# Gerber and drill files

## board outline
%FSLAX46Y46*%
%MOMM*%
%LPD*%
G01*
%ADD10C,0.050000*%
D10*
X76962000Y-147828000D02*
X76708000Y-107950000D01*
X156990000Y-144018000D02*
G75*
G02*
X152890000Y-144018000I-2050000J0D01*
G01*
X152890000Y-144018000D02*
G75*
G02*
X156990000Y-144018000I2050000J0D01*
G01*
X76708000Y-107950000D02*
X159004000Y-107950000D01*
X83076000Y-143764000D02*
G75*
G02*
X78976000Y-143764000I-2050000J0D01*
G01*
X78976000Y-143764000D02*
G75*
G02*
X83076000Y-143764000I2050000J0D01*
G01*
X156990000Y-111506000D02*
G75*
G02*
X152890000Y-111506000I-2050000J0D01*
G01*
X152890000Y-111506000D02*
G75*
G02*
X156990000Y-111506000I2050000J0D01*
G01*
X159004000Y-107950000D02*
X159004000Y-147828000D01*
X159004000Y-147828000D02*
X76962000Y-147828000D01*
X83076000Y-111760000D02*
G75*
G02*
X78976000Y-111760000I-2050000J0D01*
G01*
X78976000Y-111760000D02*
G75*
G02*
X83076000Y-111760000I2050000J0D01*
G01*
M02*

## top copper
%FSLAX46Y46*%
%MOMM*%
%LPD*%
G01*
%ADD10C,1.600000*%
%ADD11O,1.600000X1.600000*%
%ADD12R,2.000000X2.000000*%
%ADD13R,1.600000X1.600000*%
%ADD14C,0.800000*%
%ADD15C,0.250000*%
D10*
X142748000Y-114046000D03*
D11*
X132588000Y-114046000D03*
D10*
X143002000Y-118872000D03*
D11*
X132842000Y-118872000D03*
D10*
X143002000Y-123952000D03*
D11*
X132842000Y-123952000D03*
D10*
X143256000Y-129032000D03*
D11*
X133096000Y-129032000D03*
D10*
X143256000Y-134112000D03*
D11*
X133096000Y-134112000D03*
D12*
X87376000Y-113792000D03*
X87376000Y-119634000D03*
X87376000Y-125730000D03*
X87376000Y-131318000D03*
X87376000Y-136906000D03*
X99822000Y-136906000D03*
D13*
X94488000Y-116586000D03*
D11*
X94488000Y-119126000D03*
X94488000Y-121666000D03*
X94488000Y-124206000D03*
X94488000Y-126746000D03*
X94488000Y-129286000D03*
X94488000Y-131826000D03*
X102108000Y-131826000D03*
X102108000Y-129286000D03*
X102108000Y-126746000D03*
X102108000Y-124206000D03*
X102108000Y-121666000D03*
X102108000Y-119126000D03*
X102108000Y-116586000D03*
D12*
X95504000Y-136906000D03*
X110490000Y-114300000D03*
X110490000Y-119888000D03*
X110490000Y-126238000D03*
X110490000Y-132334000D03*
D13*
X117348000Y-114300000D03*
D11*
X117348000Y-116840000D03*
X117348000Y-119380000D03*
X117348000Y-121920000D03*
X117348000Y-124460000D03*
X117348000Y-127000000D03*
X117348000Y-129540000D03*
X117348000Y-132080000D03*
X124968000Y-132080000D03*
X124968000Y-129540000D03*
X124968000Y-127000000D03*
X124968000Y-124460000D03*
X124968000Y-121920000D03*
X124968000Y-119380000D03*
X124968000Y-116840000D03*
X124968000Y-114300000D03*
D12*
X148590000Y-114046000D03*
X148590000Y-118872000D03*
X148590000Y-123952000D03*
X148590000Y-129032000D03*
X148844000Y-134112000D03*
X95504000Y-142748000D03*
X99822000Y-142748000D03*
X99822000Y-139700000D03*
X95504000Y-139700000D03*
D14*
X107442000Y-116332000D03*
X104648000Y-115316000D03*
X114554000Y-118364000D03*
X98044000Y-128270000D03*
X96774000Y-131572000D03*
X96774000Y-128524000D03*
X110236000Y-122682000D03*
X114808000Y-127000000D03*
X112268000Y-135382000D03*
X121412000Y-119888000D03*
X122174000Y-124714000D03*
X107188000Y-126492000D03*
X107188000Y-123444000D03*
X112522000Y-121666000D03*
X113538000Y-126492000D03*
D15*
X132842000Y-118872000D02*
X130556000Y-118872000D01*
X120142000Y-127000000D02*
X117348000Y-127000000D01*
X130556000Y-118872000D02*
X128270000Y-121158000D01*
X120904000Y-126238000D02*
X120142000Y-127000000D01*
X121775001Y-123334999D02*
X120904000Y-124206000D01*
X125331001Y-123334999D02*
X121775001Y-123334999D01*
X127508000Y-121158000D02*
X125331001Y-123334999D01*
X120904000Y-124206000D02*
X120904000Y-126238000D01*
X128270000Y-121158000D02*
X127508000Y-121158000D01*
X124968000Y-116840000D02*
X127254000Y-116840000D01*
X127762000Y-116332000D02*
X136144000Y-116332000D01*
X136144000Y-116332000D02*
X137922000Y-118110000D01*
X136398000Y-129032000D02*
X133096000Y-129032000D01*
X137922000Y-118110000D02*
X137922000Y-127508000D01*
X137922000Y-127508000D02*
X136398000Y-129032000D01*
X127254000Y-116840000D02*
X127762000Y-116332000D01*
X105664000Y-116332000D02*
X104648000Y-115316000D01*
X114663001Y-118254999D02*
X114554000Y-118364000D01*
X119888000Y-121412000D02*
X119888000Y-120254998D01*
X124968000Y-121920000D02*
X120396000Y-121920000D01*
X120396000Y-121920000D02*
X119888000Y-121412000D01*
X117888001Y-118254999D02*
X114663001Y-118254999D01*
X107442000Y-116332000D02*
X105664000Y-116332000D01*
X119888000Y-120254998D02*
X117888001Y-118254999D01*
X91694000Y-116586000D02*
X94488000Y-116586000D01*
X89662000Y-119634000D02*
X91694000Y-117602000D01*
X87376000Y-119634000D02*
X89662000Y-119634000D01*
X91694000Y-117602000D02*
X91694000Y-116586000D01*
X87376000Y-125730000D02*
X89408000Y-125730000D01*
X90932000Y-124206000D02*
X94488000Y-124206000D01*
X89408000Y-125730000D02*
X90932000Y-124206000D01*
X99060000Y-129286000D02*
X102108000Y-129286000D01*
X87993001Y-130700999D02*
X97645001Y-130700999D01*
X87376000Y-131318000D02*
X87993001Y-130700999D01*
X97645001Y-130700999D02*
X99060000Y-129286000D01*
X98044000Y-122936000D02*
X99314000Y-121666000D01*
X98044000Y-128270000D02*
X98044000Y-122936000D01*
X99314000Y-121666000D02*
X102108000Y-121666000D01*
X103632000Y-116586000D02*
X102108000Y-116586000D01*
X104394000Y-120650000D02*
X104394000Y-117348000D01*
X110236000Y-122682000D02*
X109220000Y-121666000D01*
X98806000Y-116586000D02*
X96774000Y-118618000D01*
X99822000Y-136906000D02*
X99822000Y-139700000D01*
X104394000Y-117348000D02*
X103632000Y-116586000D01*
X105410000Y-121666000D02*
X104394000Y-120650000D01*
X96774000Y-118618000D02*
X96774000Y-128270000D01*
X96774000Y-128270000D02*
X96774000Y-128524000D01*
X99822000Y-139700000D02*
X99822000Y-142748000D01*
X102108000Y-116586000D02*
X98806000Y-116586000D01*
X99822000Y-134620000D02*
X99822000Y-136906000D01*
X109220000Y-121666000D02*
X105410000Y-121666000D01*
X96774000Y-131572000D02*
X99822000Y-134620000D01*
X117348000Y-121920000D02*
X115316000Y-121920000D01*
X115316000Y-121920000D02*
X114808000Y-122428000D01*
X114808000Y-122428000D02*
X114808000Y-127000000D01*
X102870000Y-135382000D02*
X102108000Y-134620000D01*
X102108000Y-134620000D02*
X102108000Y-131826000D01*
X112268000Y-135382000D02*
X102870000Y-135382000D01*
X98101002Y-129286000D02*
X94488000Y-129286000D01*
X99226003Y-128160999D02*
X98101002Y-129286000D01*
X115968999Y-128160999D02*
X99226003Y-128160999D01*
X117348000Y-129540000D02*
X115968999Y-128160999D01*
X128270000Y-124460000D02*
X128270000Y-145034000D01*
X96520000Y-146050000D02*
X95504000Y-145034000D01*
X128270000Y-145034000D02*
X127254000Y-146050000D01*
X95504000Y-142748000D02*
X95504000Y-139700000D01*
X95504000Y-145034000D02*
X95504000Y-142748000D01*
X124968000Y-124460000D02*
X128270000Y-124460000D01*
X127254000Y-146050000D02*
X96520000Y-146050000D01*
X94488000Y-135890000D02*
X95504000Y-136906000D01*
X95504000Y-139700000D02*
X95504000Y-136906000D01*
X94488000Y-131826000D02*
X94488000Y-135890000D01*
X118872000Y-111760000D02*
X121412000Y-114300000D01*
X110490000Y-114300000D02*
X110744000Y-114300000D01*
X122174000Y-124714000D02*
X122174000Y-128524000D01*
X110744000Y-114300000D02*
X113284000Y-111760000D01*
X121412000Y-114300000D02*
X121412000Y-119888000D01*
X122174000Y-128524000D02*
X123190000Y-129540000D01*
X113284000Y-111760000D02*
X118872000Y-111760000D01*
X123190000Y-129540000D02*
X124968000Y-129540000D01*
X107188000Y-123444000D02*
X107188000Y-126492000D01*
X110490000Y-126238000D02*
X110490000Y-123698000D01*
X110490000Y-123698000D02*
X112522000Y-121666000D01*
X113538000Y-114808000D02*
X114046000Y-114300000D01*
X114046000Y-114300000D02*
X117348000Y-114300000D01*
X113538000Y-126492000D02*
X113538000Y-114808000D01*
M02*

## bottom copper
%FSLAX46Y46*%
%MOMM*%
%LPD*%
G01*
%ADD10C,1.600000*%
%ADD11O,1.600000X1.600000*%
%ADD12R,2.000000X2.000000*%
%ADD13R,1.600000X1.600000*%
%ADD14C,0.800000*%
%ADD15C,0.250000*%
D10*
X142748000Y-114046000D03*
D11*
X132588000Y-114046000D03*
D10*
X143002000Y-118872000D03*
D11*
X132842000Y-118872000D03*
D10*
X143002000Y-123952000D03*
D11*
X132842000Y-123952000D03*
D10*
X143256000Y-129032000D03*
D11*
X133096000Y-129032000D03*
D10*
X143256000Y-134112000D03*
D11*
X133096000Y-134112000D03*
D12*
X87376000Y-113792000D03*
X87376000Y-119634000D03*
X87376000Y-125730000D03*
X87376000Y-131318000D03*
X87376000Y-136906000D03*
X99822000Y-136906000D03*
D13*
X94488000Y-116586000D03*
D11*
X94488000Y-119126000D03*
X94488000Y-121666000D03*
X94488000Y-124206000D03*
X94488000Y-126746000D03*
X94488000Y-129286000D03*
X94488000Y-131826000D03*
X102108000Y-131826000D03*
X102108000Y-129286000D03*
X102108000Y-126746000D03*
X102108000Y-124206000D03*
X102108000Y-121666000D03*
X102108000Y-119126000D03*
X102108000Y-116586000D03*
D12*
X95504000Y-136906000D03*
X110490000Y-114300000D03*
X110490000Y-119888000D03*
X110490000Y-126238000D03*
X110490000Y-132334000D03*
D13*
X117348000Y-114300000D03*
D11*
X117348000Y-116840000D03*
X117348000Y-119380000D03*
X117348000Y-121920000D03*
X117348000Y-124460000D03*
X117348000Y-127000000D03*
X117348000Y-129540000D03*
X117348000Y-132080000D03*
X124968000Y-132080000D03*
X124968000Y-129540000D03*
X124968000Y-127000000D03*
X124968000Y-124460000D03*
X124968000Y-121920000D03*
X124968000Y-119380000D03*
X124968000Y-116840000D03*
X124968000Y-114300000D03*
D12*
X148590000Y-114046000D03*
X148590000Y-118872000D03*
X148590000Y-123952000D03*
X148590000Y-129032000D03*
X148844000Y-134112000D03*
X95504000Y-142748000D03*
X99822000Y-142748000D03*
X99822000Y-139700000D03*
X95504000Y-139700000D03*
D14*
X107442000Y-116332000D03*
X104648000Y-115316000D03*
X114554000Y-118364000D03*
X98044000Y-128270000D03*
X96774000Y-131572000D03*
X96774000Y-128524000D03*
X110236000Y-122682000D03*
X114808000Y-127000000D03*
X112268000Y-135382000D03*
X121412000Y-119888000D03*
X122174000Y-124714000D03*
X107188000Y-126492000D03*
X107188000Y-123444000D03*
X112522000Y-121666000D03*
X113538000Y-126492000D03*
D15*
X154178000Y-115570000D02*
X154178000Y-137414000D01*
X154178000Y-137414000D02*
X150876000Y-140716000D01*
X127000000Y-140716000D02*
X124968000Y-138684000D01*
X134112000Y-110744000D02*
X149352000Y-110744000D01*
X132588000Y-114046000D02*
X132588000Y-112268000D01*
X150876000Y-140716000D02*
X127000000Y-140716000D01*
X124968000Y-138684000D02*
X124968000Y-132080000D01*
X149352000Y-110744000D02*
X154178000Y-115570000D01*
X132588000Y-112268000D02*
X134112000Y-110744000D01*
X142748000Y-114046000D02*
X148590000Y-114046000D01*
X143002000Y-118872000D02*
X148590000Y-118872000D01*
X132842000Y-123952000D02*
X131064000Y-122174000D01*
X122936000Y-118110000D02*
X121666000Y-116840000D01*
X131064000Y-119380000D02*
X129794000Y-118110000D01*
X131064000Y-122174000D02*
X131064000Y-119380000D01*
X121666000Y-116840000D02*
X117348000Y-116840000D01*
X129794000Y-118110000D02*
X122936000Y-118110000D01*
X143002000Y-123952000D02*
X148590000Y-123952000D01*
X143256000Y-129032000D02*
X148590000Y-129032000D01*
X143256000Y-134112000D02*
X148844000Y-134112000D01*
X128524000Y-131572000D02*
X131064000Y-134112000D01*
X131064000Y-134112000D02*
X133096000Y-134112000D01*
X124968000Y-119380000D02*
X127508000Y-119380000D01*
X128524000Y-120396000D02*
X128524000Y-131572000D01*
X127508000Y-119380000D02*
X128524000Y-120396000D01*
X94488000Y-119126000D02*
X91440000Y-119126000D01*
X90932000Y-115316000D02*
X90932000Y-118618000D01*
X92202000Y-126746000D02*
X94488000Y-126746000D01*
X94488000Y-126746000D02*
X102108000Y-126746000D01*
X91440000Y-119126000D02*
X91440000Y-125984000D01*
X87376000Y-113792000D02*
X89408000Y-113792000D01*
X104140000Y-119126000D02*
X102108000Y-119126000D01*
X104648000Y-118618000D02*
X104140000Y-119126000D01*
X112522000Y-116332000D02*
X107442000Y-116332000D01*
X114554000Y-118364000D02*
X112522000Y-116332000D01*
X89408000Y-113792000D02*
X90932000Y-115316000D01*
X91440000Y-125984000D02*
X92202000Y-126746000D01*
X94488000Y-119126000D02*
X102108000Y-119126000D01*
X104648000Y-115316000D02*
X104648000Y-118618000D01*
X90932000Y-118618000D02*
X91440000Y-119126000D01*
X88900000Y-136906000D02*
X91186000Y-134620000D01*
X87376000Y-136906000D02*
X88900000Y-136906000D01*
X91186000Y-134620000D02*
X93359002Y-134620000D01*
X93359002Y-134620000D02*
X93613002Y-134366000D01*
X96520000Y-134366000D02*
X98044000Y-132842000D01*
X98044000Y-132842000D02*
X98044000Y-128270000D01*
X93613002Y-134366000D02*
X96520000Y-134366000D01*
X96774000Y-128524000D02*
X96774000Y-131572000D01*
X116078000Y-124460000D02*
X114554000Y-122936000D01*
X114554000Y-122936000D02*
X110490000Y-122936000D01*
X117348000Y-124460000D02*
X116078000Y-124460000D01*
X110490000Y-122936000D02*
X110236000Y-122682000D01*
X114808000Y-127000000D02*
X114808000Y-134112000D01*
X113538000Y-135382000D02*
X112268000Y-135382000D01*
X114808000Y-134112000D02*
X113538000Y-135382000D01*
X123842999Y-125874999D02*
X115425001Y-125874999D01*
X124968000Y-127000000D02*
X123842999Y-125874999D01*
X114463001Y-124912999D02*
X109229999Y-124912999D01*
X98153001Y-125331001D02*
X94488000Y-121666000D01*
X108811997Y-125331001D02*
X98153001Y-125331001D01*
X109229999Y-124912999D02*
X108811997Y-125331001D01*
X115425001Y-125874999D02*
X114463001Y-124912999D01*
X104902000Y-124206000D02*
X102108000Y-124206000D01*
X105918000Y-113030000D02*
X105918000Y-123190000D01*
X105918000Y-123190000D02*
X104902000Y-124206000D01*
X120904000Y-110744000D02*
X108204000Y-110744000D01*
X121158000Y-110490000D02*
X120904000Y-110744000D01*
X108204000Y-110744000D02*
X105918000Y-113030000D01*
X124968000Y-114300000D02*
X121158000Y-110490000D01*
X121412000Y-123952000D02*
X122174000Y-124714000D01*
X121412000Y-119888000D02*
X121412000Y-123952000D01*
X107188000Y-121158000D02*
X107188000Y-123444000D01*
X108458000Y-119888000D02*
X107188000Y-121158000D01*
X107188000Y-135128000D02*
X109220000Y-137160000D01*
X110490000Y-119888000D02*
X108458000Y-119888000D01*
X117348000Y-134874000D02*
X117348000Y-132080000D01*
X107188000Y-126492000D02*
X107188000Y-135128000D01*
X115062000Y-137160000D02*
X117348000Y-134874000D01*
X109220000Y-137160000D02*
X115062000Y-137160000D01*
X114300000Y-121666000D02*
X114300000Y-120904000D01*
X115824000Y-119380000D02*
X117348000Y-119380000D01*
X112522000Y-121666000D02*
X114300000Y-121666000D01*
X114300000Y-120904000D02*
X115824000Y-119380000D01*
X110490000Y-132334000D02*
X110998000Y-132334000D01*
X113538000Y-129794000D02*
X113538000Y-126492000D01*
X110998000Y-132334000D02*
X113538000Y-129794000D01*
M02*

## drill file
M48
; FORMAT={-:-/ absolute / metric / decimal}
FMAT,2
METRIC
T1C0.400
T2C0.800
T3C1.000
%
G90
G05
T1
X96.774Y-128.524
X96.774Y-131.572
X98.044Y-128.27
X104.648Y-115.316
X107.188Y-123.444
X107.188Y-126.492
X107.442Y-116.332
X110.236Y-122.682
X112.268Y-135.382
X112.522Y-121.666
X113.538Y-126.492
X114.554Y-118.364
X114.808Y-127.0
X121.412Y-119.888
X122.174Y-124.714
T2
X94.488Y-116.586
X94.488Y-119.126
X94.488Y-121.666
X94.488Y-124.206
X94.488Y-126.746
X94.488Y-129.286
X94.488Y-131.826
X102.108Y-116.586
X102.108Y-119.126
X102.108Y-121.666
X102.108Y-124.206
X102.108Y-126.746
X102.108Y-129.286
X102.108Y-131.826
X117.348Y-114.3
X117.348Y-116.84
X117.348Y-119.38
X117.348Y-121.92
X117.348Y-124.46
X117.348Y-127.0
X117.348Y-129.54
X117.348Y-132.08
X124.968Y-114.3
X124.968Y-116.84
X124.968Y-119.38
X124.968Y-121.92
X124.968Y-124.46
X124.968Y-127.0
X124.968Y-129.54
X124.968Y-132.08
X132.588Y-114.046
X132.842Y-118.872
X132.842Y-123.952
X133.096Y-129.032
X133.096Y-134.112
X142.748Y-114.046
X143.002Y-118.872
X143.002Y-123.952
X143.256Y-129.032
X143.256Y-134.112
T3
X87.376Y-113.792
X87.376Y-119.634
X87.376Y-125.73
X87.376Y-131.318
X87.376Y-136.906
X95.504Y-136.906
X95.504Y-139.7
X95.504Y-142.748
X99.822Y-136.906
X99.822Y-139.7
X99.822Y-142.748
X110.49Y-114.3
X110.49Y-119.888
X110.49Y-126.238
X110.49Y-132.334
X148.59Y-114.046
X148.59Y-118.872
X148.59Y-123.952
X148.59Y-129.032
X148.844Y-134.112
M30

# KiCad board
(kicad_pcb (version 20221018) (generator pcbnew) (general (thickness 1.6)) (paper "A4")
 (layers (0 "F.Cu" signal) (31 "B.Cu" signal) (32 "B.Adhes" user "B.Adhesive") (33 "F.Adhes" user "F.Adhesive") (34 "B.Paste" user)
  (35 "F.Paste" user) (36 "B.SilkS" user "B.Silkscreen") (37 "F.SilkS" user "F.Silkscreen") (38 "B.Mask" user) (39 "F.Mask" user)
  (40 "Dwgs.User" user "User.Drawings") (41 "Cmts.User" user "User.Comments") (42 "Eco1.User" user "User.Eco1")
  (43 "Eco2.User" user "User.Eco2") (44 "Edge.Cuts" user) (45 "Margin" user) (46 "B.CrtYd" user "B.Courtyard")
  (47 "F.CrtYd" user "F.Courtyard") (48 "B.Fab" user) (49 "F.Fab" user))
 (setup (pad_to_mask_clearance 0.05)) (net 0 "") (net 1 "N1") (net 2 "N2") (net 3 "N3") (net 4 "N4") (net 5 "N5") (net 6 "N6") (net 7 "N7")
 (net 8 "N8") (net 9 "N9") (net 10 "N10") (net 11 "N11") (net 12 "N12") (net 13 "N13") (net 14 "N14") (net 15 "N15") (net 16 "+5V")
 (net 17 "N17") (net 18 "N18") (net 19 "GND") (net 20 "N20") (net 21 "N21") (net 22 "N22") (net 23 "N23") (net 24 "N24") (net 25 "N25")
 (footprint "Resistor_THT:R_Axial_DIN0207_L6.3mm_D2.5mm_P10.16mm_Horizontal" (layer "F.Cu") (at 142.748 114.046 180)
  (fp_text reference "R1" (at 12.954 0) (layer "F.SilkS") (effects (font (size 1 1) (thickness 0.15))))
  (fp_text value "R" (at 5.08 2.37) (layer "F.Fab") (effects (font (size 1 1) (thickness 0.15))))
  (pad "1" thru_hole circle (at 0 0 180) (size 1.6 1.6) (drill 0.8) (layers "*.Cu" "*.Mask") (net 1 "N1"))
  (pad "2" thru_hole oval (at 10.16 0 180) (size 1.6 1.6) (drill 0.8) (layers "*.Cu" "*.Mask") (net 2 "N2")))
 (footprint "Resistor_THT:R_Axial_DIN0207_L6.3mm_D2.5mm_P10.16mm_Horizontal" (layer "F.Cu") (at 143.002 118.872 180)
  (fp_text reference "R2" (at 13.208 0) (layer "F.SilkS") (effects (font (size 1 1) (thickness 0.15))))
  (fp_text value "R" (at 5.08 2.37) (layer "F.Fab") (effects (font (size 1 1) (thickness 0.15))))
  (pad "1" thru_hole circle (at 0 0 180) (size 1.6 1.6) (drill 0.8) (layers "*.Cu" "*.Mask") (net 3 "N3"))
  (pad "2" thru_hole oval (at 10.16 0 180) (size 1.6 1.6) (drill 0.8) (layers "*.Cu" "*.Mask") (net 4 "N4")))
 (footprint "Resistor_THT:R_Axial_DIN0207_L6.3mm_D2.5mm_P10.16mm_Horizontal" (layer "F.Cu") (at 143.002 123.952 180)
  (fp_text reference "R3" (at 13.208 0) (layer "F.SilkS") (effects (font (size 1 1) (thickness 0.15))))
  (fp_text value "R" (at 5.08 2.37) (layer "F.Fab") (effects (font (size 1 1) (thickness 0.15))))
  (pad "1" thru_hole circle (at 0 0 180) (size 1.6 1.6) (drill 0.8) (layers "*.Cu" "*.Mask") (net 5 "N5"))
  (pad "2" thru_hole oval (at 10.16 0 180) (size 1.6 1.6) (drill 0.8) (layers "*.Cu" "*.Mask") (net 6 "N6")))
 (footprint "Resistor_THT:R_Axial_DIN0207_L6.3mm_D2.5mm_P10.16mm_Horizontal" (layer "F.Cu") (at 143.256 129.032 180)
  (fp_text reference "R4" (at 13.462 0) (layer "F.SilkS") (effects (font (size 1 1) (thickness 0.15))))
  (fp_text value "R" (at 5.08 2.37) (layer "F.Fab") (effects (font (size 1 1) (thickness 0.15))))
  (pad "1" thru_hole circle (at 0 0 180) (size 1.6 1.6) (drill 0.8) (layers "*.Cu" "*.Mask") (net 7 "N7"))
  (pad "2" thru_hole oval (at 10.16 0 180) (size 1.6 1.6) (drill 0.8) (layers "*.Cu" "*.Mask") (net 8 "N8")))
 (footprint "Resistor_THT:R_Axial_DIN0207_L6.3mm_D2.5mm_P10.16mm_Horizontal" (layer "F.Cu") (at 143.256 134.112 180)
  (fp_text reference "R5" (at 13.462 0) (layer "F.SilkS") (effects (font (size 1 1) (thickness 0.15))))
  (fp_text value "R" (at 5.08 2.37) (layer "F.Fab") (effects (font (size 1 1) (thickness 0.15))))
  (pad "1" thru_hole circle (at 0 0 180) (size 1.6 1.6) (drill 0.8) (layers "*.Cu" "*.Mask") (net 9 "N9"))
  (pad "2" thru_hole oval (at 10.16 0 180) (size 1.6 1.6) (drill 0.8) (layers "*.Cu" "*.Mask") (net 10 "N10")))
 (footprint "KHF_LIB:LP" (layer "F.Cu") (at 87.376 113.792)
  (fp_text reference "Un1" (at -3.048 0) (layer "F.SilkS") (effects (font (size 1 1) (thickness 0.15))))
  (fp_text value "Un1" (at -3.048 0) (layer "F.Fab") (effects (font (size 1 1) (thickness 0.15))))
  (pad "1" thru_hole rect (at 0 0) (size 2 2) (drill 1) (layers "*.Cu" "*.Mask") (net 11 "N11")))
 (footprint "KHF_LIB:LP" (layer "F.Cu") (at 87.376 119.634)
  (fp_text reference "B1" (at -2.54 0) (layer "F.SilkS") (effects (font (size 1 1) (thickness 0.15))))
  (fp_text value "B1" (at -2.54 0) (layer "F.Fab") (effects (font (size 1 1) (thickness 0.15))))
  (pad "1" thru_hole rect (at 0 0) (size 2 2) (drill 1) (layers "*.Cu" "*.Mask") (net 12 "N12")))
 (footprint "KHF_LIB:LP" (layer "F.Cu") (at 87.376 125.73)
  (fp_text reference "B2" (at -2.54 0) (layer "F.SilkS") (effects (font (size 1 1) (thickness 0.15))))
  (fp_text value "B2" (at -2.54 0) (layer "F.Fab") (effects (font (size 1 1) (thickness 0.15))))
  (pad "1" thru_hole rect (at 0 0) (size 2 2) (drill 1) (layers "*.Cu" "*.Mask") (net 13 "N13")))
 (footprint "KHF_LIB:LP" (layer "F.Cu") (at 87.376 131.318)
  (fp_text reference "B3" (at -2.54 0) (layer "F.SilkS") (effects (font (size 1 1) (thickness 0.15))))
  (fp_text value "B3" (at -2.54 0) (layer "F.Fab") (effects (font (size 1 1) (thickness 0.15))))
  (pad "1" thru_hole rect (at 0 0) (size 2 2) (drill 1) (layers "*.Cu" "*.Mask") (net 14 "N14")))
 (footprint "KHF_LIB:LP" (layer "F.Cu") (at 87.376 136.906)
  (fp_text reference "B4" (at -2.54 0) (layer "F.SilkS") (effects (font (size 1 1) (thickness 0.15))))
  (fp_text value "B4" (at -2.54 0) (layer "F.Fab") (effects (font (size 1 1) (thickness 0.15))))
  (pad "1" thru_hole rect (at 0 0) (size 2 2) (drill 1) (layers "*.Cu" "*.Mask") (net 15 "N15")))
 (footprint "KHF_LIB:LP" (layer "F.Cu") (at 99.822 136.906)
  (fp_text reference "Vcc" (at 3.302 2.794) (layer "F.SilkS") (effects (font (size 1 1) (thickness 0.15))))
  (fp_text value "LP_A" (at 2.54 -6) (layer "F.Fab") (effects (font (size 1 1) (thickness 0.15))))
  (pad "1" thru_hole rect (at 0 0) (size 2 2) (drill 1) (layers "*.Cu" "*.Mask") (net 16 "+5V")))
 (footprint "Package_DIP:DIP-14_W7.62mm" (layer "F.Cu") (at 94.488 116.586)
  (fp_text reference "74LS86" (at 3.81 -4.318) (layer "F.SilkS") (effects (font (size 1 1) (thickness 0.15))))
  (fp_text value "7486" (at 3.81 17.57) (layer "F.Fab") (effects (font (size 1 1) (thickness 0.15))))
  (pad "1" thru_hole rect (at 0 0) (size 1.6 1.6) (drill 0.8) (layers "*.Cu" "*.Mask") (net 12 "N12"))
  (pad "2" thru_hole oval (at 0 2.54) (size 1.6 1.6) (drill 0.8) (layers "*.Cu" "*.Mask") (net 11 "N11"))
  (pad "3" thru_hole oval (at 0 5.08) (size 1.6 1.6) (drill 0.8) (layers "*.Cu" "*.Mask") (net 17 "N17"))
  (pad "4" thru_hole oval (at 0 7.62) (size 1.6 1.6) (drill 0.8) (layers "*.Cu" "*.Mask") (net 13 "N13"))
  (pad "5" thru_hole oval (at 0 10.16) (size 1.6 1.6) (drill 0.8) (layers "*.Cu" "*.Mask") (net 11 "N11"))
  (pad "6" thru_hole oval (at 0 12.7) (size 1.6 1.6) (drill 0.8) (layers "*.Cu" "*.Mask") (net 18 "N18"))
  (pad "7" thru_hole oval (at 0 15.24) (size 1.6 1.6) (drill 0.8) (layers "*.Cu" "*.Mask") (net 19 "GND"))
  (pad "8" thru_hole oval (at 7.62 15.24) (size 1.6 1.6) (drill 0.8) (layers "*.Cu" "*.Mask") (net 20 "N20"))
  (pad "9" thru_hole oval (at 7.62 12.7) (size 1.6 1.6) (drill 0.8) (layers "*.Cu" "*.Mask") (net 14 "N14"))
  (pad "10" thru_hole oval (at 7.62 10.16) (size 1.6 1.6) (drill 0.8) (layers "*.Cu" "*.Mask") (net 11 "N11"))
  (pad "11" thru_hole oval (at 7.62 7.62) (size 1.6 1.6) (drill 0.8) (layers "*.Cu" "*.Mask") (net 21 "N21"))
  (pad "12" thru_hole oval (at 7.62 5.08) (size 1.6 1.6) (drill 0.8) (layers "*.Cu" "*.Mask") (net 15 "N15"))
  (pad "13" thru_hole oval (at 7.62 2.54) (size 1.6 1.6) (drill 0.8) (layers "*.Cu" "*.Mask") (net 11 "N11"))
  (pad "14" thru_hole oval (at 7.62 0) (size 1.6 1.6) (drill 0.8) (layers "*.Cu" "*.Mask") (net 16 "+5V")))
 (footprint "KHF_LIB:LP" (layer "F.Cu") (at 95.504 136.906)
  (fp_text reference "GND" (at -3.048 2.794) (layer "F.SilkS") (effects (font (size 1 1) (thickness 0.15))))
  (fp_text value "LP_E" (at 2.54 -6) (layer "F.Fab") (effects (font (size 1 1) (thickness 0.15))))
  (pad "1" thru_hole rect (at 0 0) (size 2 2) (drill 1) (layers "*.Cu" "*.Mask") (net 19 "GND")))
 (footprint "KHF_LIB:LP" (layer "F.Cu") (at 110.49 114.3)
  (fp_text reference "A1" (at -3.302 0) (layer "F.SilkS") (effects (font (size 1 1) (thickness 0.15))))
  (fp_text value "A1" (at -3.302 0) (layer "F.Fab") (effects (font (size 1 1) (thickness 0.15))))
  (pad "1" thru_hole rect (at 0 0) (size 2 2) (drill 1) (layers "*.Cu" "*.Mask") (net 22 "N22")))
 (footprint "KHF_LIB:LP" (layer "F.Cu") (at 110.49 119.888)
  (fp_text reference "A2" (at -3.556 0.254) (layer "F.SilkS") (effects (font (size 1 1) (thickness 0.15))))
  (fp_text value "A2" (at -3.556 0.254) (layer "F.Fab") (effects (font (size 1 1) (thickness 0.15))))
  (pad "1" thru_hole rect (at 0 0) (size 2 2) (drill 1) (layers "*.Cu" "*.Mask") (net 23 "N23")))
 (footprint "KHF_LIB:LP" (layer "F.Cu") (at 110.49 126.238)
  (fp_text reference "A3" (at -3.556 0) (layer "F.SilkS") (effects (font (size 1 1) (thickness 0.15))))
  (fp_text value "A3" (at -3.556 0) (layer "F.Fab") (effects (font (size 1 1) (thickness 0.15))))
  (pad "1" thru_hole rect (at 0 0) (size 2 2) (drill 1) (layers "*.Cu" "*.Mask") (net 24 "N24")))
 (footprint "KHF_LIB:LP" (layer "F.Cu") (at 110.49 132.334)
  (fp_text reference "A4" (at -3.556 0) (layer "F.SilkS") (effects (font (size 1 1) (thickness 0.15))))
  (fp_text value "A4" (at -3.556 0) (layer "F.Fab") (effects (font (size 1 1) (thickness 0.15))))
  (pad "1" thru_hole rect (at 0 0) (size 2 2) (drill 1) (layers "*.Cu" "*.Mask") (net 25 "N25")))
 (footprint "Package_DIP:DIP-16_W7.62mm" (layer "F.Cu") (at 117.348 114.3)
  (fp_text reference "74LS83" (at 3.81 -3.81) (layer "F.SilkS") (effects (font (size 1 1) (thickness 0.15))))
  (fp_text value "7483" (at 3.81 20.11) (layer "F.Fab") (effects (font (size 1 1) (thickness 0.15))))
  (pad "1" thru_hole rect (at 0 0) (size 1.6 1.6) (drill 0.8) (layers "*.Cu" "*.Mask") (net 25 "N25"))
  (pad "2" thru_hole oval (at 0 2.54) (size 1.6 1.6) (drill 0.8) (layers "*.Cu" "*.Mask") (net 6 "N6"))
  (pad "3" thru_hole oval (at 0 5.08) (size 1.6 1.6) (drill 0.8) (layers "*.Cu" "*.Mask") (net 24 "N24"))
  (pad "4" thru_hole oval (at 0 7.62) (size 1.6 1.6) (drill 0.8) (layers "*.Cu" "*.Mask") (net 20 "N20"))
  (pad "5" thru_hole oval (at 0 10.16) (size 1.6 1.6) (drill 0.8) (layers "*.Cu" "*.Mask") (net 16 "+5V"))
  (pad "6" thru_hole oval (at 0 12.7) (size 1.6 1.6) (drill 0.8) (layers "*.Cu" "*.Mask") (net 4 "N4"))
  (pad "7" thru_hole oval (at 0 15.24) (size 1.6 1.6) (drill 0.8) (layers "*.Cu" "*.Mask") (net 18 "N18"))
  (pad "8" thru_hole oval (at 0 17.78) (size 1.6 1.6) (drill 0.8) (layers "*.Cu" "*.Mask") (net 23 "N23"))
  (pad "9" thru_hole oval (at 7.62 17.78) (size 1.6 1.6) (drill 0.8) (layers "*.Cu" "*.Mask") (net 2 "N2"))
  (pad "10" thru_hole oval (at 7.62 15.24) (size 1.6 1.6) (drill 0.8) (layers "*.Cu" "*.Mask") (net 22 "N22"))
  (pad "11" thru_hole oval (at 7.62 12.7) (size 1.6 1.6) (drill 0.8) (layers "*.Cu" "*.Mask") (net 17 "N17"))
  (pad "12" thru_hole oval (at 7.62 10.16) (size 1.6 1.6) (drill 0.8) (layers "*.Cu" "*.Mask") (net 19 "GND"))
  (pad "13" thru_hole oval (at 7.62 7.62) (size 1.6 1.6) (drill 0.8) (layers "*.Cu" "*.Mask") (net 11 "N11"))
  (pad "14" thru_hole oval (at 7.62 5.08) (size 1.6 1.6) (drill 0.8) (layers "*.Cu" "*.Mask") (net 10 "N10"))
  (pad "15" thru_hole oval (at 7.62 2.54) (size 1.6 1.6) (drill 0.8) (layers "*.Cu" "*.Mask") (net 8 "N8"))
  (pad "16" thru_hole oval (at 7.62 0) (size 1.6 1.6) (drill 0.8) (layers "*.Cu" "*.Mask") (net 21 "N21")))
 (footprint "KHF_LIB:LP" (layer "F.Cu") (at 148.59 114.046)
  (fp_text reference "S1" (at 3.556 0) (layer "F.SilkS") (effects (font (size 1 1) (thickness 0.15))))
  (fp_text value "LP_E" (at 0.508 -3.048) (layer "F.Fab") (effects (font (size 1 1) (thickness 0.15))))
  (pad "1" thru_hole rect (at 0 0) (size 2 2) (drill 1) (layers "*.Cu" "*.Mask") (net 1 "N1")))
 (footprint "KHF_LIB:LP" (layer "F.Cu") (at 148.59 118.872)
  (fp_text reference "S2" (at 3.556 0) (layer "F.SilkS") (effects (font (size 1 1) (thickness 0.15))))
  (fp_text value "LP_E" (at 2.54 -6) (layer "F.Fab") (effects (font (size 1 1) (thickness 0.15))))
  (pad "1" thru_hole rect (at 0 0) (size 2 2) (drill 1) (layers "*.Cu" "*.Mask") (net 3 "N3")))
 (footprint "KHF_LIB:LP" (layer "F.Cu") (at 148.59 123.952)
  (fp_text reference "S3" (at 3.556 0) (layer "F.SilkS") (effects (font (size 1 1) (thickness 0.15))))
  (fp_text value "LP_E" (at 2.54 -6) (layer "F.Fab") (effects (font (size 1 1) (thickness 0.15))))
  (pad "1" thru_hole rect (at 0 0) (size 2 2) (drill 1) (layers "*.Cu" "*.Mask") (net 5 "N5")))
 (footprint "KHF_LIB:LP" (layer "F.Cu") (at 148.59 129.032)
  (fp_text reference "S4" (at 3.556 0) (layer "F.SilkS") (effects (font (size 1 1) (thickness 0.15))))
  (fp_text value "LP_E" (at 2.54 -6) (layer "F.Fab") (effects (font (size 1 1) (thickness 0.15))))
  (pad "1" thru_hole rect (at 0 0) (size 2 2) (drill 1) (layers "*.Cu" "*.Mask") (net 7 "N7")))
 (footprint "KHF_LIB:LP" (layer "F.Cu") (at 148.844 134.112)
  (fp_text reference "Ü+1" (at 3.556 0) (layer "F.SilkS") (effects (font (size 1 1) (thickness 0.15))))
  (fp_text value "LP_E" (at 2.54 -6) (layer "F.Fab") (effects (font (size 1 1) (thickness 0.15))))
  (pad "1" thru_hole rect (at 0 0) (size 2 2) (drill 1) (layers "*.Cu" "*.Mask") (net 9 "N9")))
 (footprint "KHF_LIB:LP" (layer "F.Cu") (at 95.504 142.748)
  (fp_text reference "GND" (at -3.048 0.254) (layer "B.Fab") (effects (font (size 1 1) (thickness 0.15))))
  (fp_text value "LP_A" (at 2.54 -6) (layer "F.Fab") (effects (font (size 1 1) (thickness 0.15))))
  (pad "1" thru_hole rect (at 0 0) (size 2 2) (drill 1) (layers "*.Cu" "*.Mask") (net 19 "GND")))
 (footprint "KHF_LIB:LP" (layer "F.Cu") (at 99.822 142.748)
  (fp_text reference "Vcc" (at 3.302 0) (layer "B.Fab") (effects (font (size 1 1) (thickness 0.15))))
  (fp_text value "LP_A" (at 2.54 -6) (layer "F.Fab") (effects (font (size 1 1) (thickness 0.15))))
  (pad "1" thru_hole rect (at 0 0) (size 2 2) (drill 1) (layers "*.Cu" "*.Mask") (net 16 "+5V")))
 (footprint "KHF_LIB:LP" (layer "F.Cu") (at 99.822 139.7)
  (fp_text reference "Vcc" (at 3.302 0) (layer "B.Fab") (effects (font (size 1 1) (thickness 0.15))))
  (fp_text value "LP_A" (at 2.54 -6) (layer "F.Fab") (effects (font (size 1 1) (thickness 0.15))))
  (pad "1" thru_hole rect (at 0 0) (size 2 2) (drill 1) (layers "*.Cu" "*.Mask") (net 16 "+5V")))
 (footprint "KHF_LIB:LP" (layer "F.Cu") (at 95.504 139.7)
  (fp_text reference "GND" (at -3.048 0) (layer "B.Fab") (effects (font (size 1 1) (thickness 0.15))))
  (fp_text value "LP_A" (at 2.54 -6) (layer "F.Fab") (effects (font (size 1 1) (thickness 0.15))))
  (pad "1" thru_hole rect (at 0 0) (size 2 2) (drill 1) (layers "*.Cu" "*.Mask") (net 19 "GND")))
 (gr_line (start 76.962 147.828) (end 76.708 107.95) (stroke (width 0.05) (type solid)) (layer "Edge.Cuts"))
 (gr_circle (center 154.94 144.018) (end 156.99 144.018) (stroke (width 0.05) (type solid)) (fill none) (layer "Edge.Cuts"))
 (gr_line (start 76.708 107.95) (end 159.004 107.95) (stroke (width 0.05) (type solid)) (layer "Edge.Cuts"))
 (gr_circle (center 81.026 143.764) (end 83.076 143.764) (stroke (width 0.05) (type solid)) (fill none) (layer "Edge.Cuts"))
 (gr_circle (center 154.94 111.506) (end 156.99 111.506) (stroke (width 0.05) (type solid)) (fill none) (layer "Edge.Cuts"))
 (gr_line (start 159.004 107.95) (end 159.004 147.828) (stroke (width 0.05) (type solid)) (layer "Edge.Cuts"))
 (gr_line (start 159.004 147.828) (end 76.962 147.828) (stroke (width 0.05) (type solid)) (layer "Edge.Cuts"))
 (gr_circle (center 81.026 111.76) (end 83.076 111.76) (stroke (width 0.05) (type solid)) (fill none) (layer "Edge.Cuts"))
 (segment (start 154.178 115.57) (end 154.178 137.414) (width 0.25) (layer "B.Cu") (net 2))
 (segment (start 154.178 137.414) (end 150.876 140.716) (width 0.25) (layer "B.Cu") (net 2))
 (segment (start 127 140.716) (end 124.968 138.684) (width 0.25) (layer "B.Cu") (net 2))
 (segment (start 134.112 110.744) (end 149.352 110.744) (width 0.25) (layer "B.Cu") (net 2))
 (segment (start 132.588 114.046) (end 132.588 112.268) (width 0.25) (layer "B.Cu") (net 2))
 (segment (start 150.876 140.716) (end 127 140.716) (width 0.25) (layer "B.Cu") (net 2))
 (segment (start 124.968 138.684) (end 124.968 132.08) (width 0.25) (layer "B.Cu") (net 2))
 (segment (start 149.352 110.744) (end 154.178 115.57) (width 0.25) (layer "B.Cu") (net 2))
 (segment (start 132.588 112.268) (end 134.112 110.744) (width 0.25) (layer "B.Cu") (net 2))
 (segment (start 142.748 114.046) (end 148.59 114.046) (width 0.25) (layer "B.Cu") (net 1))
 (segment (start 143.002 118.872) (end 148.59 118.872) (width 0.25) (layer "B.Cu") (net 3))
 (segment (start 132.842 118.872) (end 130.556 118.872) (width 0.25) (layer "F.Cu") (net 4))
 (segment (start 120.142 127) (end 117.348 127) (width 0.25) (layer "F.Cu") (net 4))
 (segment (start 130.556 118.872) (end 128.27 121.158) (width 0.25) (layer "F.Cu") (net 4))
 (segment (start 120.904 126.238) (end 120.142 127) (width 0.25) (layer "F.Cu") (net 4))
 (segment (start 121.775001 123.334999) (end 120.904 124.206) (width 0.25) (layer "F.Cu") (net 4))
 (segment (start 125.331001 123.334999) (end 121.775001 123.334999) (width 0.25) (layer "F.Cu") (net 4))
 (segment (start 127.508 121.158) (end 125.331001 123.334999) (width 0.25) (layer "F.Cu") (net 4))
 (segment (start 120.904 124.206) (end 120.904 126.238) (width 0.25) (layer "F.Cu") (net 4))
 (segment (start 128.27 121.158) (end 127.508 121.158) (width 0.25) (layer "F.Cu") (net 4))
 (segment (start 132.842 123.952) (end 131.064 122.174) (width 0.25) (layer "B.Cu") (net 6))
 (segment (start 122.936 118.11) (end 121.666 116.84) (width 0.25) (layer "B.Cu") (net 6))
 (segment (start 131.064 119.38) (end 129.794 118.11) (width 0.25) (layer "B.Cu") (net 6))
 (segment (start 131.064 122.174) (end 131.064 119.38) (width 0.25) (layer "B.Cu") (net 6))
 (segment (start 121.666 116.84) (end 117.348 116.84) (width 0.25) (layer "B.Cu") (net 6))
 (segment (start 129.794 118.11) (end 122.936 118.11) (width 0.25) (layer "B.Cu") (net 6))
 (segment (start 143.002 123.952) (end 148.59 123.952) (width 0.25) (layer "B.Cu") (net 5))
 (segment (start 143.256 129.032) (end 148.59 129.032) (width 0.25) (layer "B.Cu") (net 7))
 (segment (start 124.968 116.84) (end 127.254 116.84) (width 0.25) (layer "F.Cu") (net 8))
 (segment (start 127.762 116.332) (end 136.144 116.332) (width 0.25) (layer "F.Cu") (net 8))
 (segment (start 136.144 116.332) (end 137.922 118.11) (width 0.25) (layer "F.Cu") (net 8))
 (segment (start 136.398 129.032) (end 133.096 129.032) (width 0.25) (layer "F.Cu") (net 8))
 (segment (start 137.922 118.11) (end 137.922 127.508) (width 0.25) (layer "F.Cu") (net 8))
 (segment (start 137.922 127.508) (end 136.398 129.032) (width 0.25) (layer "F.Cu") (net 8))
 (segment (start 127.254 116.84) (end 127.762 116.332) (width 0.25) (layer "F.Cu") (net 8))
 (segment (start 143.256 134.112) (end 148.844 134.112) (width 0.25) (layer "B.Cu") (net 9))
 (segment (start 128.524 131.572) (end 131.064 134.112) (width 0.25) (layer "B.Cu") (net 10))
 (segment (start 131.064 134.112) (end 133.096 134.112) (width 0.25) (layer "B.Cu") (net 10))
 (segment (start 124.968 119.38) (end 127.508 119.38) (width 0.25) (layer "B.Cu") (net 10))
 (segment (start 128.524 120.396) (end 128.524 131.572) (width 0.25) (layer "B.Cu") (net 10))
 (segment (start 127.508 119.38) (end 128.524 120.396) (width 0.25) (layer "B.Cu") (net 10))
 (segment (start 105.664 116.332) (end 104.648 115.316) (width 0.25) (layer "F.Cu") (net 11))
 (segment (start 114.663001 118.254999) (end 114.554 118.364) (width 0.25) (layer "F.Cu") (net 11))
 (segment (start 119.888 121.412) (end 119.888 120.254998) (width 0.25) (layer "F.Cu") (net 11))
 (segment (start 124.968 121.92) (end 120.396 121.92) (width 0.25) (layer "F.Cu") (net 11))
 (segment (start 120.396 121.92) (end 119.888 121.412) (width 0.25) (layer "F.Cu") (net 11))
 (segment (start 117.888001 118.254999) (end 114.663001 118.254999) (width 0.25) (layer "F.Cu") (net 11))
 (segment (start 107.442 116.332) (end 105.664 116.332) (width 0.25) (layer "F.Cu") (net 11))
 (segment (start 119.888 120.254998) (end 117.888001 118.254999) (width 0.25) (layer "F.Cu") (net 11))
 (via (at 107.442 116.332) (size 0.8) (drill 0.4) (layers "F.Cu" "B.Cu") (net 11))
 (via (at 104.648 115.316) (size 0.8) (drill 0.4) (layers "F.Cu" "B.Cu") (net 11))
 (via (at 114.554 118.364) (size 0.8) (drill 0.4) (layers "F.Cu" "B.Cu") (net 11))
 (segment (start 94.488 119.126) (end 91.44 119.126) (width 0.25) (layer "B.Cu") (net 11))
 (segment (start 90.932 115.316) (end 90.932 118.618) (width 0.25) (layer "B.Cu") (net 11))
 (segment (start 92.202 126.746) (end 94.488 126.746) (width 0.25) (layer "B.Cu") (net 11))
 (segment (start 94.488 126.746) (end 102.108 126.746) (width 0.25) (layer "B.Cu") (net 11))
 (segment (start 91.44 119.126) (end 91.44 125.984) (width 0.25) (layer "B.Cu") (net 11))
 (segment (start 87.376 113.792) (end 89.408 113.792) (width 0.25) (layer "B.Cu") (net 11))
 (segment (start 104.14 119.126) (end 102.108 119.126) (width 0.25) (layer "B.Cu") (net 11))
 (segment (start 104.648 118.618) (end 104.14 119.126) (width 0.25) (layer "B.Cu") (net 11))
 (segment (start 112.522 116.332) (end 107.442 116.332) (width 0.25) (layer "B.Cu") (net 11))
 (segment (start 114.554 118.364) (end 112.522 116.332) (width 0.25) (layer "B.Cu") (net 11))
 (segment (start 89.408 113.792) (end 90.932 115.316) (width 0.25) (layer "B.Cu") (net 11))
 (segment (start 91.44 125.984) (end 92.202 126.746) (width 0.25) (layer "B.Cu") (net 11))
 (segment (start 94.488 119.126) (end 102.108 119.126) (width 0.25) (layer "B.Cu") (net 11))
 (segment (start 104.648 115.316) (end 104.648 118.618) (width 0.25) (layer "B.Cu") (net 11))
 (segment (start 90.932 118.618) (end 91.44 119.126) (width 0.25) (layer "B.Cu") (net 11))
 (segment (start 91.694 116.586) (end 94.488 116.586) (width 0.25) (layer "F.Cu") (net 12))
 (segment (start 89.662 119.634) (end 91.694 117.602) (width 0.25) (layer "F.Cu") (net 12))
 (segment (start 87.376 119.634) (end 89.662 119.634) (width 0.25) (layer "F.Cu") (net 12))
 (segment (start 91.694 117.602) (end 91.694 116.586) (width 0.25) (layer "F.Cu") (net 12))
 (segment (start 87.376 125.73) (end 89.408 125.73) (width 0.25) (layer "F.Cu") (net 13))
 (segment (start 90.932 124.206) (end 94.488 124.206) (width 0.25) (layer "F.Cu") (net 13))
 (segment (start 89.408 125.73) (end 90.932 124.206) (width 0.25) (layer "F.Cu") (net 13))
 (segment (start 99.06 129.286) (end 102.108 129.286) (width 0.25) (layer "F.Cu") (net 14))
 (segment (start 87.993001 130.700999) (end 97.645001 130.700999) (width 0.25) (layer "F.Cu") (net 14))
 (segment (start 87.376 131.318) (end 87.993001 130.700999) (width 0.25) (layer "F.Cu") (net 14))
 (segment (start 97.645001 130.700999) (end 99.06 129.286) (width 0.25) (layer "F.Cu") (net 14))
 (segment (start 98.044 122.936) (end 99.314 121.666) (width 0.25) (layer "F.Cu") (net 15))
 (segment (start 98.044 128.27) (end 98.044 122.936) (width 0.25) (layer "F.Cu") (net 15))
 (segment (start 99.314 121.666) (end 102.108 121.666) (width 0.25) (layer "F.Cu") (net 15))
 (via (at 98.044 128.27) (size 0.8) (drill 0.4) (layers "F.Cu" "B.Cu") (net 15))
 (segment (start 88.9 136.906) (end 91.186 134.62) (width 0.25) (layer "B.Cu") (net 15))
 (segment (start 87.376 136.906) (end 88.9 136.906) (width 0.25) (layer "B.Cu") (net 15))
 (segment (start 91.186 134.62) (end 93.359002 134.62) (width 0.25) (layer "B.Cu") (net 15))
 (segment (start 93.359002 134.62) (end 93.613002 134.366) (width 0.25) (layer "B.Cu") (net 15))
 (segment (start 96.52 134.366) (end 98.044 132.842) (width 0.25) (layer "B.Cu") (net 15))
 (segment (start 98.044 132.842) (end 98.044 128.27) (width 0.25) (layer "B.Cu") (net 15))
 (segment (start 93.613002 134.366) (end 96.52 134.366) (width 0.25) (layer "B.Cu") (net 15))
 (segment (start 103.632 116.586) (end 102.108 116.586) (width 0.25) (layer "F.Cu") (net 16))
 (segment (start 104.394 120.65) (end 104.394 117.348) (width 0.25) (layer "F.Cu") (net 16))
 (segment (start 110.236 122.682) (end 109.22 121.666) (width 0.25) (layer "F.Cu") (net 16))
 (segment (start 98.806 116.586) (end 96.774 118.618) (width 0.25) (layer "F.Cu") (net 16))
 (segment (start 99.822 136.906) (end 99.822 139.7) (width 0.25) (layer "F.Cu") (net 16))
 (segment (start 104.394 117.348) (end 103.632 116.586) (width 0.25) (layer "F.Cu") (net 16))
 (segment (start 105.41 121.666) (end 104.394 120.65) (width 0.25) (layer "F.Cu") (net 16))
 (segment (start 96.774 118.618) (end 96.774 128.27) (width 0.25) (layer "F.Cu") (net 16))
 (segment (start 96.774 128.27) (end 96.774 128.524) (width 0.25) (layer "F.Cu") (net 16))
 (segment (start 99.822 139.7) (end 99.822 142.748) (width 0.25) (layer "F.Cu") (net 16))
 (segment (start 102.108 116.586) (end 98.806 116.586) (width 0.25) (layer "F.Cu") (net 16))
 (segment (start 99.822 134.62) (end 99.822 136.906) (width 0.25) (layer "F.Cu") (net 16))
 (segment (start 109.22 121.666) (end 105.41 121.666) (width 0.25) (layer "F.Cu") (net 16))
 (segment (start 96.774 131.572) (end 99.822 134.62) (width 0.25) (layer "F.Cu") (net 16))
 (via (at 96.774 131.572) (size 0.8) (drill 0.4) (layers "F.Cu" "B.Cu") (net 16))
 (via (at 96.774 128.524) (size 0.8) (drill 0.4) (layers "F.Cu" "B.Cu") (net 16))
 (via (at 110.236 122.682) (size 0.8) (drill 0.4) (layers "F.Cu" "B.Cu") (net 16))
 (segment (start 96.774 128.524) (end 96.774 131.572) (width 0.25) (layer "B.Cu") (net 16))
 (segment (start 116.078 124.46) (end 114.554 122.936) (width 0.25) (layer "B.Cu") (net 16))
 (segment (start 114.554 122.936) (end 110.49 122.936) (width 0.25) (layer "B.Cu") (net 16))
 (segment (start 117.348 124.46) (end 116.078 124.46) (width 0.25) (layer "B.Cu") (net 16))
 (segment (start 110.49 122.936) (end 110.236 122.682) (width 0.25) (layer "B.Cu") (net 16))
 (segment (start 117.348 121.92) (end 115.316 121.92) (width 0.25) (layer "F.Cu") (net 20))
 (segment (start 115.316 121.92) (end 114.808 122.428) (width 0.25) (layer "F.Cu") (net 20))
 (segment (start 114.808 122.428) (end 114.808 127) (width 0.25) (layer "F.Cu") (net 20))
 (segment (start 102.87 135.382) (end 102.108 134.62) (width 0.25) (layer "F.Cu") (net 20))
 (segment (start 102.108 134.62) (end 102.108 131.826) (width 0.25) (layer "F.Cu") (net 20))
 (segment (start 112.268 135.382) (end 102.87 135.382) (width 0.25) (layer "F.Cu") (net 20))
 (via (at 114.808 127) (size 0.8) (drill 0.4) (layers "F.Cu" "B.Cu") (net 20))
 (via (at 112.268 135.382) (size 0.8) (drill 0.4) (layers "F.Cu" "B.Cu") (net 20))
 (segment (start 114.808 127) (end 114.808 134.112) (width 0.25) (layer "B.Cu") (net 20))
 (segment (start 113.538 135.382) (end 112.268 135.382) (width 0.25) (layer "B.Cu") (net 20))
 (segment (start 114.808 134.112) (end 113.538 135.382) (width 0.25) (layer "B.Cu") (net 20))
 (segment (start 123.842999 125.874999) (end 115.425001 125.874999) (width 0.25) (layer "B.Cu") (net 17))
 (segment (start 124.968 127) (end 123.842999 125.874999) (width 0.25) (layer "B.Cu") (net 17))
 (segment (start 114.463001 124.912999) (end 109.229999 124.912999) (width 0.25) (layer "B.Cu") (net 17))
 (segment (start 98.153001 125.331001) (end 94.488 121.666) (width 0.25) (layer "B.Cu") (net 17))
 (segment (start 108.811997 125.331001) (end 98.153001 125.331001) (width 0.25) (layer "B.Cu") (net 17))
 (segment (start 109.229999 124.912999) (end 108.811997 125.331001) (width 0.25) (layer "B.Cu") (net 17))
 (segment (start 115.425001 125.874999) (end 114.463001 124.912999) (width 0.25) (layer "B.Cu") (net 17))
 (segment (start 104.902 124.206) (end 102.108 124.206) (width 0.25) (layer "B.Cu") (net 21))
 (segment (start 105.918 113.03) (end 105.918 123.19) (width 0.25) (layer "B.Cu") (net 21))
 (segment (start 105.918 123.19) (end 104.902 124.206) (width 0.25) (layer "B.Cu") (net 21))
 (segment (start 120.904 110.744) (end 108.204 110.744) (width 0.25) (layer "B.Cu") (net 21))
 (segment (start 121.158 110.49) (end 120.904 110.744) (width 0.25) (layer "B.Cu") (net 21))
 (segment (start 108.204 110.744) (end 105.918 113.03) (width 0.25) (layer "B.Cu") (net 21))
 (segment (start 124.968 114.3) (end 121.158 110.49) (width 0.25) (layer "B.Cu") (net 21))
 (segment (start 98.101002 129.286) (end 94.488 129.286) (width 0.25) (layer "F.Cu") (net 18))
 (segment (start 99.226003 128.160999) (end 98.101002 129.286) (width 0.25) (layer "F.Cu") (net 18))
 (segment (start 115.968999 128.160999) (end 99.226003 128.160999) (width 0.25) (layer "F.Cu") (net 18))
 (segment (start 117.348 129.54) (end 115.968999 128.160999) (width 0.25) (layer "F.Cu") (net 18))
 (segment (start 128.27 124.46) (end 128.27 145.034) (width 0.25) (layer "F.Cu") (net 19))
 (segment (start 96.52 146.05) (end 95.504 145.034) (width 0.25) (layer "F.Cu") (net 19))
 (segment (start 128.27 145.034) (end 127.254 146.05) (width 0.25) (layer "F.Cu") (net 19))
 (segment (start 95.504 142.748) (end 95.504 139.7) (width 0.25) (layer "F.Cu") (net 19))
 (segment (start 95.504 145.034) (end 95.504 142.748) (width 0.25) (layer "F.Cu") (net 19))
 (segment (start 124.968 124.46) (end 128.27 124.46) (width 0.25) (layer "F.Cu") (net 19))
 (segment (start 127.254 146.05) (end 96.52 146.05) (width 0.25) (layer "F.Cu") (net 19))
 (segment (start 94.488 135.89) (end 95.504 136.906) (width 0.25) (layer "F.Cu") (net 19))
 (segment (start 95.504 139.7) (end 95.504 136.906) (width 0.25) (layer "F.Cu") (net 19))
 (segment (start 94.488 131.826) (end 94.488 135.89) (width 0.25) (layer "F.Cu") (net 19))
 (segment (start 118.872 111.76) (end 121.412 114.3) (width 0.25) (layer "F.Cu") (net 22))
 (segment (start 110.49 114.3) (end 110.744 114.3) (width 0.25) (layer "F.Cu") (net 22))
 (segment (start 122.174 124.714) (end 122.174 128.524) (width 0.25) (layer "F.Cu") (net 22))
 (segment (start 110.744 114.3) (end 113.284 111.76) (width 0.25) (layer "F.Cu") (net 22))
 (segment (start 121.412 114.3) (end 121.412 119.888) (width 0.25) (layer "F.Cu") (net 22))
 (segment (start 122.174 128.524) (end 123.19 129.54) (width 0.25) (layer "F.Cu") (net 22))
 (segment (start 113.284 111.76) (end 118.872 111.76) (width 0.25) (layer "F.Cu") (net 22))
 (segment (start 123.19 129.54) (end 124.968 129.54) (width 0.25) (layer "F.Cu") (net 22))
 (via (at 121.412 119.888) (size 0.8) (drill 0.4) (layers "F.Cu" "B.Cu") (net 22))
 (via (at 122.174 124.714) (size 0.8) (drill 0.4) (layers "F.Cu" "B.Cu") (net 22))
 (segment (start 121.412 123.952) (end 122.174 124.714) (width 0.25) (layer "B.Cu") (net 22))
 (segment (start 121.412 119.888) (end 121.412 123.952) (width 0.25) (layer "B.Cu") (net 22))
 (segment (start 107.188 123.444) (end 107.188 126.492) (width 0.25) (layer "F.Cu") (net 23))
 (via (at 107.188 126.492) (size 0.8) (drill 0.4) (layers "F.Cu" "B.Cu") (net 23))
 (via (at 107.188 123.444) (size 0.8) (drill 0.4) (layers "F.Cu" "B.Cu") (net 23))
 (segment (start 107.188 121.158) (end 107.188 123.444) (width 0.25) (layer "B.Cu") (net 23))
 (segment (start 108.458 119.888) (end 107.188 121.158) (width 0.25) (layer "B.Cu") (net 23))
 (segment (start 107.188 135.128) (end 109.22 137.16) (width 0.25) (layer "B.Cu") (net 23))
 (segment (start 110.49 119.888) (end 108.458 119.888) (width 0.25) (layer "B.Cu") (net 23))
 (segment (start 117.348 134.874) (end 117.348 132.08) (width 0.25) (layer "B.Cu") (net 23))
 (segment (start 107.188 126.492) (end 107.188 135.128) (width 0.25) (layer "B.Cu") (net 23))
 (segment (start 115.062 137.16) (end 117.348 134.874) (width 0.25) (layer "B.Cu") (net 23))
 (segment (start 109.22 137.16) (end 115.062 137.16) (width 0.25) (layer "B.Cu") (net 23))
 (segment (start 110.49 126.238) (end 110.49 123.698) (width 0.25) (layer "F.Cu") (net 24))
 (segment (start 110.49 123.698) (end 112.522 121.666) (width 0.25) (layer "F.Cu") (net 24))
 (via (at 112.522 121.666) (size 0.8) (drill 0.4) (layers "F.Cu" "B.Cu") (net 24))
 (segment (start 114.3 121.666) (end 114.3 120.904) (width 0.25) (layer "B.Cu") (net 24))
 (segment (start 115.824 119.38) (end 117.348 119.38) (width 0.25) (layer "B.Cu") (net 24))
 (segment (start 112.522 121.666) (end 114.3 121.666) (width 0.25) (layer "B.Cu") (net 24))
 (segment (start 114.3 120.904) (end 115.824 119.38) (width 0.25) (layer "B.Cu") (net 24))
 (segment (start 113.538 114.808) (end 114.046 114.3) (width 0.25) (layer "F.Cu") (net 25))
 (segment (start 114.046 114.3) (end 117.348 114.3) (width 0.25) (layer "F.Cu") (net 25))
 (segment (start 113.538 126.492) (end 113.538 114.808) (width 0.25) (layer "F.Cu") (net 25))
 (via (at 113.538 126.492) (size 0.8) (drill 0.4) (layers "F.Cu" "B.Cu") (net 25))
 (segment (start 110.49 132.334) (end 110.998 132.334) (width 0.25) (layer "B.Cu") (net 25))
 (segment (start 113.538 129.794) (end 113.538 126.492) (width 0.25) (layer "B.Cu") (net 25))
 (segment (start 110.998 132.334) (end 113.538 129.794) (width 0.25) (layer "B.Cu") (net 25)))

